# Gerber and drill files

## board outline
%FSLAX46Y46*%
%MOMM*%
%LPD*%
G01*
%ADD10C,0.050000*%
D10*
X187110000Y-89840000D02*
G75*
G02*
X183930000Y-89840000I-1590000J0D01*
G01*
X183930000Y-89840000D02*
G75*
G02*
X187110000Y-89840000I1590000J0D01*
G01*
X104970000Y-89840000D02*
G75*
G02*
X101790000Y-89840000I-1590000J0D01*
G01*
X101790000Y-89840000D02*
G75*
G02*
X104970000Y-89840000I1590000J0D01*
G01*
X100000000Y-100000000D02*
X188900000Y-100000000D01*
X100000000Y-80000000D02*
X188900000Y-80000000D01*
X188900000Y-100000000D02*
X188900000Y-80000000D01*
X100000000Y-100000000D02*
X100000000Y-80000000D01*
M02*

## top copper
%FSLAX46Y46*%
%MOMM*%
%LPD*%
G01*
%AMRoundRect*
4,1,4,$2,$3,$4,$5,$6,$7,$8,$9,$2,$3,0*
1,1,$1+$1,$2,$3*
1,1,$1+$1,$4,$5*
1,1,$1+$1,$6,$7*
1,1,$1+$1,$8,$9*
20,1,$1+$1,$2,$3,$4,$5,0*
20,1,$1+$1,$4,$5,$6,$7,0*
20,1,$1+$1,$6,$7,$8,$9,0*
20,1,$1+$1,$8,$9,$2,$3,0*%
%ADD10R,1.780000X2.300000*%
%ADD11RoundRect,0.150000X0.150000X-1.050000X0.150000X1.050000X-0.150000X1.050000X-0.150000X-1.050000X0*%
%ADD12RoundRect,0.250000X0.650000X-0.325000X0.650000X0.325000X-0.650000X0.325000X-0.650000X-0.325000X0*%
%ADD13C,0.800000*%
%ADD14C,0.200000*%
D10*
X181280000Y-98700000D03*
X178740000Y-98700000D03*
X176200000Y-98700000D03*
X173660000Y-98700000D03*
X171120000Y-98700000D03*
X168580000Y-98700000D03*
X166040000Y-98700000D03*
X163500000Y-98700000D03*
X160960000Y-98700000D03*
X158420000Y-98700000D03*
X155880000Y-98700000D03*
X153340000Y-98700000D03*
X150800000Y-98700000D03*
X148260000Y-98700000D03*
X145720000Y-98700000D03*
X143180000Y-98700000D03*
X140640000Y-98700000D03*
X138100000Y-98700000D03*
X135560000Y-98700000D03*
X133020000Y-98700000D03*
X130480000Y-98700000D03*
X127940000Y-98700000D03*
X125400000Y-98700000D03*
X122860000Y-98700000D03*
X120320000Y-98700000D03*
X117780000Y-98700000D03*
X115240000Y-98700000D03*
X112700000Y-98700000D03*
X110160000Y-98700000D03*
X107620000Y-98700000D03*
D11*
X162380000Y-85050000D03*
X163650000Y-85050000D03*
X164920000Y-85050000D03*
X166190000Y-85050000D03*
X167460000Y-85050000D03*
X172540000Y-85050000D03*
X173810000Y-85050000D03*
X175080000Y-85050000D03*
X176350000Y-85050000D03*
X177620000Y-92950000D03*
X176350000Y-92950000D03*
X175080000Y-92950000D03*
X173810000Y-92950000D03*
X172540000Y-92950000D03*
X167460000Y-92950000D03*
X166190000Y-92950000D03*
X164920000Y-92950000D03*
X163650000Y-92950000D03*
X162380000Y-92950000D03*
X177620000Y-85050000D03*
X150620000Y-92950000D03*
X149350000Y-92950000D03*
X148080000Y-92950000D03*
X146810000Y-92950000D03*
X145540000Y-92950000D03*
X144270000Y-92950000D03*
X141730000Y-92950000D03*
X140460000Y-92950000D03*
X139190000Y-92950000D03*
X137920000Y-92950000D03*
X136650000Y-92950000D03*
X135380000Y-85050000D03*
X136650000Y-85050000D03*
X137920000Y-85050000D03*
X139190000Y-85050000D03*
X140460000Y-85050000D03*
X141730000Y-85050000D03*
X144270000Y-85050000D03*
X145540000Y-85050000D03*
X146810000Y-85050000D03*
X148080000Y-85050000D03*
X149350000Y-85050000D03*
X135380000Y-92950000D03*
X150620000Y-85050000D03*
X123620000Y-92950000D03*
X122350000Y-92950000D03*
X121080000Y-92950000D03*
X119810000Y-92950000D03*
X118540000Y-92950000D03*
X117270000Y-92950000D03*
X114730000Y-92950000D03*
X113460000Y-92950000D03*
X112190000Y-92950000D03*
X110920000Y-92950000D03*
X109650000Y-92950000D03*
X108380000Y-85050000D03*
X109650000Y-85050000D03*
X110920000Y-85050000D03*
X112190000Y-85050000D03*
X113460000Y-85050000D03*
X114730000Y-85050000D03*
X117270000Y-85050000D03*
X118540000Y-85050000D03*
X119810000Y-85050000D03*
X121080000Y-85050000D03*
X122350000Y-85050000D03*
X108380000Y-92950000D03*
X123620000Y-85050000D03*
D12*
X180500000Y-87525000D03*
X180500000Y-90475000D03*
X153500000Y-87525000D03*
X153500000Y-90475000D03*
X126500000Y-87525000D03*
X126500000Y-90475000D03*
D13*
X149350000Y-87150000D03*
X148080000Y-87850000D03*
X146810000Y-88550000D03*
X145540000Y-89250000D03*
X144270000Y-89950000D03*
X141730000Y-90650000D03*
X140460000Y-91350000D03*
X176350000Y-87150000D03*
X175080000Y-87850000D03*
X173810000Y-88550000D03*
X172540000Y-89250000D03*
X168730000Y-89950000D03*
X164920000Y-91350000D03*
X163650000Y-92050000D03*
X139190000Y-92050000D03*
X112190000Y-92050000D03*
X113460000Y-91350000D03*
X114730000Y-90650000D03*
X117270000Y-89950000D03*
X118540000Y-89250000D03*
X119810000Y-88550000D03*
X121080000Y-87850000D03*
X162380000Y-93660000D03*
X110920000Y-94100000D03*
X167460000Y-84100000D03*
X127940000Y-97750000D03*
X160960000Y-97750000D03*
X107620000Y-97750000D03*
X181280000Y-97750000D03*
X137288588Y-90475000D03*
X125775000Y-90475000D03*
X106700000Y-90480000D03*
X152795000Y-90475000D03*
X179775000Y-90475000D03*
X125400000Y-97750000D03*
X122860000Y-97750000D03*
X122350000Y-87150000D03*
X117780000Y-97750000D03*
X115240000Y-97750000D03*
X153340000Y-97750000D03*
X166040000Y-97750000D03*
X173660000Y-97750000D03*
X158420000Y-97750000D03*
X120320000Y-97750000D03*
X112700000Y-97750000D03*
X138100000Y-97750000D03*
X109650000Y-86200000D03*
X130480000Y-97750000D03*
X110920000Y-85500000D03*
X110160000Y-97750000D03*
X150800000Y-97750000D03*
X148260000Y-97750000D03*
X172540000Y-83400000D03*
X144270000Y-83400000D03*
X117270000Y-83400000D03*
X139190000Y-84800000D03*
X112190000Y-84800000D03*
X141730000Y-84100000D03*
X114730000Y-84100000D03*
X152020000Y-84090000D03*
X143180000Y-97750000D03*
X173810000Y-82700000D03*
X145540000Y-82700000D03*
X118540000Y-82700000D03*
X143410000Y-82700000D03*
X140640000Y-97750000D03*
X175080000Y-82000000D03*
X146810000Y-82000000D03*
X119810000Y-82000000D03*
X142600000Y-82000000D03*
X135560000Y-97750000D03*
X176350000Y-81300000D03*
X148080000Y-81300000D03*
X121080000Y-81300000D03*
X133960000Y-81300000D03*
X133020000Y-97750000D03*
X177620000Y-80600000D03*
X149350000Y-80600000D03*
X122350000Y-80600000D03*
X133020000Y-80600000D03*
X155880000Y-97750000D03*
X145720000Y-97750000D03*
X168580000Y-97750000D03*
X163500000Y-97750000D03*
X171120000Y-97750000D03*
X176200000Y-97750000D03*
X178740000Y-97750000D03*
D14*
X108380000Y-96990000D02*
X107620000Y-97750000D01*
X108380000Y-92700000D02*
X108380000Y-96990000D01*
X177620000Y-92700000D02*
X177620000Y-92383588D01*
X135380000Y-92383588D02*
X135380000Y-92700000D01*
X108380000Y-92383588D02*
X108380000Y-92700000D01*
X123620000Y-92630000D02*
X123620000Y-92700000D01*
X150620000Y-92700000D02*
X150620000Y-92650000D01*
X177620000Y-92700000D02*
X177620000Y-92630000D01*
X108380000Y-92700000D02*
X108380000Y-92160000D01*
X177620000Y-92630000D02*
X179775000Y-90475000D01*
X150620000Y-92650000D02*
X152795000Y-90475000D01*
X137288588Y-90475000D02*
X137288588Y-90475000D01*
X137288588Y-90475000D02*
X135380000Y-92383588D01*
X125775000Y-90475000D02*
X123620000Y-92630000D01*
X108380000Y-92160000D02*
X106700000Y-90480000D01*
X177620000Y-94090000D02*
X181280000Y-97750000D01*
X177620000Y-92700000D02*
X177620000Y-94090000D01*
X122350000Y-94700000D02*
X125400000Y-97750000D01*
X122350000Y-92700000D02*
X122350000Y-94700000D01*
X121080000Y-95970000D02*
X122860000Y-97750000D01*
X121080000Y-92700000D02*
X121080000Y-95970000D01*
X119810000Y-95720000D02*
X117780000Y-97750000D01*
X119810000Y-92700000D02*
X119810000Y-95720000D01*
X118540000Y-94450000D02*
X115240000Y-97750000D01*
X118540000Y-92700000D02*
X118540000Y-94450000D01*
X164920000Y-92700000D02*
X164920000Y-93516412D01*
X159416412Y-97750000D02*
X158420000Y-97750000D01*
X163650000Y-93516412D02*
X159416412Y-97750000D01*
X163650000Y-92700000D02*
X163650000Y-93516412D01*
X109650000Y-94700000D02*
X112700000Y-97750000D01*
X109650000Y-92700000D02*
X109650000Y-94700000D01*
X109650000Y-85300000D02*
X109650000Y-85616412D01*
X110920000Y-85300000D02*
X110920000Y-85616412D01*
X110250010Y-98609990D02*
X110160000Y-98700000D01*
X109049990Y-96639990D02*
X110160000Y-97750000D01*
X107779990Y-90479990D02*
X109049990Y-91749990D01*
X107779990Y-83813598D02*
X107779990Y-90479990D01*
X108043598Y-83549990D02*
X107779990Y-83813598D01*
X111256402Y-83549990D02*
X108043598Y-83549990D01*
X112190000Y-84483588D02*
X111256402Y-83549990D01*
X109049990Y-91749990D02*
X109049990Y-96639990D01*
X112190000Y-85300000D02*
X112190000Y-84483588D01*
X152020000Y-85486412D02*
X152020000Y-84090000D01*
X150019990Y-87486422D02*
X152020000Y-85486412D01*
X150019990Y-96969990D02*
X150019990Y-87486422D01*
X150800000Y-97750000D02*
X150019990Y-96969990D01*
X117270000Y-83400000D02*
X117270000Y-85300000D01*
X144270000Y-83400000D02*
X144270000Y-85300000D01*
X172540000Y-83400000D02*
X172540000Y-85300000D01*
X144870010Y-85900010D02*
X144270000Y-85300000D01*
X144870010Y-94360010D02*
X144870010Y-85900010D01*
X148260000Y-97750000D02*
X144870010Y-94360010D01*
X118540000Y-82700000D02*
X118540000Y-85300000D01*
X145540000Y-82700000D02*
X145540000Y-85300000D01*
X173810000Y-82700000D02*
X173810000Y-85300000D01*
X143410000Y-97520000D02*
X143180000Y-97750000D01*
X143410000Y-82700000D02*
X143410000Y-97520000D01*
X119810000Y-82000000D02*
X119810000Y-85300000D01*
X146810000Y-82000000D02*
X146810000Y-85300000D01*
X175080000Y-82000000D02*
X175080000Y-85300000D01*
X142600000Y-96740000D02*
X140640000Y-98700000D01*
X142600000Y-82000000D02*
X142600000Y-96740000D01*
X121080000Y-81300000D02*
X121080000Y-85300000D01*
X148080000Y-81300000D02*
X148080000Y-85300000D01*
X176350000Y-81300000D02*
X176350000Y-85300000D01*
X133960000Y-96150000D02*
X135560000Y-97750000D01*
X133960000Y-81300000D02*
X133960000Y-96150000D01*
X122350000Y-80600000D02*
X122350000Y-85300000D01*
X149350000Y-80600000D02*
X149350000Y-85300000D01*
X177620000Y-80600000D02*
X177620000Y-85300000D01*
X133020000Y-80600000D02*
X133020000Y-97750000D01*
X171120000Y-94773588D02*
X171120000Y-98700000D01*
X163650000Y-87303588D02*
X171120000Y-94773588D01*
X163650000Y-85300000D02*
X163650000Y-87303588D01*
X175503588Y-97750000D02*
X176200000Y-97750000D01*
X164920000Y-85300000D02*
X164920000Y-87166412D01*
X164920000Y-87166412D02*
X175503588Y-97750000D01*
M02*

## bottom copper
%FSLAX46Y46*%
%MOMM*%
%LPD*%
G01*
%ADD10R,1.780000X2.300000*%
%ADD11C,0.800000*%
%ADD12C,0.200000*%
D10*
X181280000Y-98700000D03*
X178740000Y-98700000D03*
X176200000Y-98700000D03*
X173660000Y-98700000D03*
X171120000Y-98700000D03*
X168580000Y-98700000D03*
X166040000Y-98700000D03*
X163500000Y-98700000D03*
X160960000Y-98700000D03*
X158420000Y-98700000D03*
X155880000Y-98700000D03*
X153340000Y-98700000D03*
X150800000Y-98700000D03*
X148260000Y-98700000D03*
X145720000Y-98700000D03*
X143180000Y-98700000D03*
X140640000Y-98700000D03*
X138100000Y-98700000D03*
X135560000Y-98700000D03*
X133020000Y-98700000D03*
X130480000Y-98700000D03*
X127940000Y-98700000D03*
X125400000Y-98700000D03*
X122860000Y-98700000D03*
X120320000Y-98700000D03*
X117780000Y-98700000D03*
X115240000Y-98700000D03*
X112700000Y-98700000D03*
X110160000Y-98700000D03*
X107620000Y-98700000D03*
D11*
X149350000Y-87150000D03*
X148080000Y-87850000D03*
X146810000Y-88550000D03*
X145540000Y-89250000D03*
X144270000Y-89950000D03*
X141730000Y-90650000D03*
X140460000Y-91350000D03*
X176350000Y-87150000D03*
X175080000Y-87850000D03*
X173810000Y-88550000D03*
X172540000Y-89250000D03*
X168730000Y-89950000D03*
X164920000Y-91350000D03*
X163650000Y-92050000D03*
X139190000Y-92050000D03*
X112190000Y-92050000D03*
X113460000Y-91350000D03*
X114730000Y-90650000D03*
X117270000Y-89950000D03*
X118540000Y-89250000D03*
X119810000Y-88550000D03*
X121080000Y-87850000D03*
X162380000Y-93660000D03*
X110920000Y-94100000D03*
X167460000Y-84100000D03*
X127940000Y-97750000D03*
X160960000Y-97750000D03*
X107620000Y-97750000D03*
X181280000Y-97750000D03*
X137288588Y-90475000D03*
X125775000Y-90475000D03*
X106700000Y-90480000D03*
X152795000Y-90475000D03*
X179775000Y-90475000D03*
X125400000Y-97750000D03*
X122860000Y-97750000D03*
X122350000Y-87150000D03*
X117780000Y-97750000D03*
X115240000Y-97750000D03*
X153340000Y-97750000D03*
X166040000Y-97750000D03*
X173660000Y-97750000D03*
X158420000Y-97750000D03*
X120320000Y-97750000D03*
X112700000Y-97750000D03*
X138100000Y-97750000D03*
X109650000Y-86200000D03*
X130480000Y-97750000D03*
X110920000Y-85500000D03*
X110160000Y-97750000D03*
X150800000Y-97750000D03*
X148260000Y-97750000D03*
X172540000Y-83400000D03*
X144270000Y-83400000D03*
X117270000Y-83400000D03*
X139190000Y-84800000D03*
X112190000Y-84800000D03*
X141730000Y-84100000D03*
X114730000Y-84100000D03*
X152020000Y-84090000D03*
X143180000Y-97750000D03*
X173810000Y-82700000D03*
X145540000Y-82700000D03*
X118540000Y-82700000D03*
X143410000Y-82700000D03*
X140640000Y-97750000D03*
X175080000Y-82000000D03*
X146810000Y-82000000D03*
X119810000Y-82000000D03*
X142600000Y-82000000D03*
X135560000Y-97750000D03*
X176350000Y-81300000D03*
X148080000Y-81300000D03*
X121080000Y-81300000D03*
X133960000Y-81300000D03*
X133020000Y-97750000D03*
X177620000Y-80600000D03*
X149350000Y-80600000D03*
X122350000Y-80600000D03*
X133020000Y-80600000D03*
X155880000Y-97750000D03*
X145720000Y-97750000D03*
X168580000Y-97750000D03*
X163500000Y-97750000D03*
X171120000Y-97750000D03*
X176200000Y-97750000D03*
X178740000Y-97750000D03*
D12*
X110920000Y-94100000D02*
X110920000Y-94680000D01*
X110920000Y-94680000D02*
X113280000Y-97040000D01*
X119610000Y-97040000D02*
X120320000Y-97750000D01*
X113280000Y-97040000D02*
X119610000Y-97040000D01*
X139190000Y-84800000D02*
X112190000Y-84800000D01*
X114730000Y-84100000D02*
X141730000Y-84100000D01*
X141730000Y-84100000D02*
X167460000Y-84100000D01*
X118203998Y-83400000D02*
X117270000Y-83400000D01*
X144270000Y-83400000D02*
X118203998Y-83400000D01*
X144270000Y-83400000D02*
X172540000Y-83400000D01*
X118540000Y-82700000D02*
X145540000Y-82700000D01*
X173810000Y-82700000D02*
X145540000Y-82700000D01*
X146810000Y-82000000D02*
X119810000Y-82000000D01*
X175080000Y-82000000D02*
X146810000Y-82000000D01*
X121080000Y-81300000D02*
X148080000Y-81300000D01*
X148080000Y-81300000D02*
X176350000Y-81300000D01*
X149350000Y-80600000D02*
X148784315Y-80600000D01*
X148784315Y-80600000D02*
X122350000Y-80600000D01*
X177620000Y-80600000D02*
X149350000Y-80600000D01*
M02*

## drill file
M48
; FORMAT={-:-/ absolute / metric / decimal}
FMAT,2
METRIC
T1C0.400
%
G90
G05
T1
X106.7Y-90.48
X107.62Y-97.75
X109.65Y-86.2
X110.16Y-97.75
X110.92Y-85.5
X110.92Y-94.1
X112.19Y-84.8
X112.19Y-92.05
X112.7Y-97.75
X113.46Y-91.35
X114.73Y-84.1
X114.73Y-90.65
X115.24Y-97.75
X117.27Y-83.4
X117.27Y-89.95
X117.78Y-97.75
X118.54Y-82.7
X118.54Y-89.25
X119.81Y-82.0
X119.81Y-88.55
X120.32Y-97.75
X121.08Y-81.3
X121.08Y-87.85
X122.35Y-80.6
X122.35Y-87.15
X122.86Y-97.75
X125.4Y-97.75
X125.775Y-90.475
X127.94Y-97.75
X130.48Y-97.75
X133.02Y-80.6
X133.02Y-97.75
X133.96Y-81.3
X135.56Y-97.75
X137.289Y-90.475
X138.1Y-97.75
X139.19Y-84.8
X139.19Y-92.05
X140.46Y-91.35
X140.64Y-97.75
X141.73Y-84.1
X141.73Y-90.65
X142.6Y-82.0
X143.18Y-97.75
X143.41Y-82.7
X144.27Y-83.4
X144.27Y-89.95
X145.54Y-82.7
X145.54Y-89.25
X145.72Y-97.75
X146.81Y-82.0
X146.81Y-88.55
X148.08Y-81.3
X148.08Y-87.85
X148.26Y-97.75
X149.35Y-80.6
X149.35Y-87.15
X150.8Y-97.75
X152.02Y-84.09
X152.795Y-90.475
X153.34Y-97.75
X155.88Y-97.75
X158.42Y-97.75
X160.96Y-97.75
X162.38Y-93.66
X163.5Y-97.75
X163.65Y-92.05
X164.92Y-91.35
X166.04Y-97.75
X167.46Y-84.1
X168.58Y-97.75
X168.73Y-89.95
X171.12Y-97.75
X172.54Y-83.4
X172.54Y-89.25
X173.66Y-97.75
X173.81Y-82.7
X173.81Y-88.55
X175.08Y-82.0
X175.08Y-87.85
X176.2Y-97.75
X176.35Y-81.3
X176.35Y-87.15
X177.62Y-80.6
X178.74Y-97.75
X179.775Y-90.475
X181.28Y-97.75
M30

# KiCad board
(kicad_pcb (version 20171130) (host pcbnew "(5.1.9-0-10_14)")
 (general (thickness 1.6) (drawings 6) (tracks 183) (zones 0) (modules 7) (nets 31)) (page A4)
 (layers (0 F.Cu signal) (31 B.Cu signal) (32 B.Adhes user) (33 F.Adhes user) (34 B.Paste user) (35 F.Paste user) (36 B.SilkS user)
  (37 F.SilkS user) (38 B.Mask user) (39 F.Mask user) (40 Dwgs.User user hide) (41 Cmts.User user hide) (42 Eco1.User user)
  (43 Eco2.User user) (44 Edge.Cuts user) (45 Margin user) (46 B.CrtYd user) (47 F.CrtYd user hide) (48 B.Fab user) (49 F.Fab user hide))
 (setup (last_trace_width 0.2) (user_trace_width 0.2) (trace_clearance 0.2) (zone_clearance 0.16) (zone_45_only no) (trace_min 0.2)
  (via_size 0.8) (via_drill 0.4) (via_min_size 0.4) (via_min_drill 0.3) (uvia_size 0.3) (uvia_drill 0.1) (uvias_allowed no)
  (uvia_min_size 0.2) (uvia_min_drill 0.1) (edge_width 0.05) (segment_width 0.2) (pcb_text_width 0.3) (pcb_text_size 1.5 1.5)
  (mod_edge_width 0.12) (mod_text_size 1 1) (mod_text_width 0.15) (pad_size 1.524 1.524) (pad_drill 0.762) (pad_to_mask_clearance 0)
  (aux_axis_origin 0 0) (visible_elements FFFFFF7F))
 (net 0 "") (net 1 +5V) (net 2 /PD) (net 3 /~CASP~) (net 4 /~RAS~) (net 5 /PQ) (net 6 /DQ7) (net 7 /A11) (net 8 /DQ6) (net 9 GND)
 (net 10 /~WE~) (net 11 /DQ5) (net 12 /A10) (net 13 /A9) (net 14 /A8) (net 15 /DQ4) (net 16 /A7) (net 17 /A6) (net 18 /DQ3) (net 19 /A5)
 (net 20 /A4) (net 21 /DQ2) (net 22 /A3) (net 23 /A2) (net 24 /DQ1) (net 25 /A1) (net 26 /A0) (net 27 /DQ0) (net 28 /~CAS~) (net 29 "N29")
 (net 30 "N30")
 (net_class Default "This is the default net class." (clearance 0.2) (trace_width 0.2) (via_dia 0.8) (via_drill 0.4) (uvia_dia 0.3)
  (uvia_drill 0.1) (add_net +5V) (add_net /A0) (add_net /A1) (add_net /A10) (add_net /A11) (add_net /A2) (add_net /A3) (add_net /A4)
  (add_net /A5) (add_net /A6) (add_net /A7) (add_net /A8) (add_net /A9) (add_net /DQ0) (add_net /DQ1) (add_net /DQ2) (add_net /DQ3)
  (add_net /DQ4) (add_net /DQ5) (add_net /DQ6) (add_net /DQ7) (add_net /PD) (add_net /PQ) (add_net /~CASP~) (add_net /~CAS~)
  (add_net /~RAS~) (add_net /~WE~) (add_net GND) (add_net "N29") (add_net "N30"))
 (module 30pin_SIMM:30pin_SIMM (layer F.Cu) (at 100 100)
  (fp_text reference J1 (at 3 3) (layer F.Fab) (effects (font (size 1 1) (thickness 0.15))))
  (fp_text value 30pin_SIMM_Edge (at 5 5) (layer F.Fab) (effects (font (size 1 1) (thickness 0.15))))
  (pad 30 connect rect (at 81.28 -1.3) (size 1.78 2.3) (layers B.Cu B.Mask) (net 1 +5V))
  (pad 29 connect rect (at 78.74 -1.3) (size 1.78 2.3) (layers B.Cu B.Mask) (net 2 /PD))
  (pad 28 connect rect (at 76.2 -1.3) (size 1.78 2.3) (layers B.Cu B.Mask) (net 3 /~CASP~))
  (pad 27 connect rect (at 73.66 -1.3) (size 1.78 2.3) (layers B.Cu B.Mask) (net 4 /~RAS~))
  (pad 26 connect rect (at 71.12 -1.3) (size 1.78 2.3) (layers B.Cu B.Mask) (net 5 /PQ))
  (pad 25 connect rect (at 68.58 -1.3) (size 1.78 2.3) (layers B.Cu B.Mask) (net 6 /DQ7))
  (pad 24 connect rect (at 66.04 -1.3) (size 1.78 2.3) (layers B.Cu B.Mask) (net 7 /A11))
  (pad 23 connect rect (at 63.5 -1.3) (size 1.78 2.3) (layers B.Cu B.Mask) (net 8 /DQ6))
  (pad 22 connect rect (at 60.96 -1.3) (size 1.78 2.3) (layers B.Cu B.Mask) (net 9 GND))
  (pad 21 connect rect (at 58.42 -1.3) (size 1.78 2.3) (layers B.Cu B.Mask) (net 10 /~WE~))
  (pad 20 connect rect (at 55.88 -1.3) (size 1.78 2.3) (layers B.Cu B.Mask) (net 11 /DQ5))
  (pad 19 connect rect (at 53.34 -1.3) (size 1.78 2.3) (layers B.Cu B.Mask) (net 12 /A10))
  (pad 18 connect rect (at 50.8 -1.3) (size 1.78 2.3) (layers B.Cu B.Mask) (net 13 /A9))
  (pad 17 connect rect (at 48.26 -1.3) (size 1.78 2.3) (layers B.Cu B.Mask) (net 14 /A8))
  (pad 16 connect rect (at 45.72 -1.3) (size 1.78 2.3) (layers B.Cu B.Mask) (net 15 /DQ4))
  (pad 15 connect rect (at 43.18 -1.3) (size 1.78 2.3) (layers B.Cu B.Mask) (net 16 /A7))
  (pad 14 connect rect (at 40.64 -1.3) (size 1.78 2.3) (layers B.Cu B.Mask) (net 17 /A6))
  (pad 13 connect rect (at 38.1 -1.3) (size 1.78 2.3) (layers B.Cu B.Mask) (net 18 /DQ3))
  (pad 12 connect rect (at 35.56 -1.3) (size 1.78 2.3) (layers B.Cu B.Mask) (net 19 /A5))
  (pad 11 connect rect (at 33.02 -1.3) (size 1.78 2.3) (layers B.Cu B.Mask) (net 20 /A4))
  (pad 10 connect rect (at 30.48 -1.3) (size 1.78 2.3) (layers B.Cu B.Mask) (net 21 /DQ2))
  (pad 9 connect rect (at 27.94 -1.3) (size 1.78 2.3) (layers B.Cu B.Mask) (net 9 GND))
  (pad 8 connect rect (at 25.4 -1.3) (size 1.78 2.3) (layers B.Cu B.Mask) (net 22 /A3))
  (pad 7 connect rect (at 22.86 -1.3) (size 1.78 2.3) (layers B.Cu B.Mask) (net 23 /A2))
  (pad 6 connect rect (at 20.32 -1.3) (size 1.78 2.3) (layers B.Cu B.Mask) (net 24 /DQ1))
  (pad 5 connect rect (at 17.78 -1.3) (size 1.78 2.3) (layers B.Cu B.Mask) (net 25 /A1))
  (pad 4 connect rect (at 15.24 -1.3) (size 1.78 2.3) (layers B.Cu B.Mask) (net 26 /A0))
  (pad 3 connect rect (at 12.7 -1.3) (size 1.78 2.3) (layers B.Cu B.Mask) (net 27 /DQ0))
  (pad 2 connect rect (at 10.16 -1.3) (size 1.78 2.3) (layers B.Cu B.Mask) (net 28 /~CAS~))
  (pad 30 connect rect (at 81.28 -1.3) (size 1.78 2.3) (layers F.Cu F.Mask) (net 1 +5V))
  (pad 29 connect rect (at 78.74 -1.3) (size 1.78 2.3) (layers F.Cu F.Mask) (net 2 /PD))
  (pad 28 connect rect (at 76.2 -1.3) (size 1.78 2.3) (layers F.Cu F.Mask) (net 3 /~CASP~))
  (pad 27 connect rect (at 73.66 -1.3) (size 1.78 2.3) (layers F.Cu F.Mask) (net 4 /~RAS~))
  (pad 26 connect rect (at 71.12 -1.3) (size 1.78 2.3) (layers F.Cu F.Mask) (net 5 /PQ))
  (pad 25 connect rect (at 68.58 -1.3) (size 1.78 2.3) (layers F.Cu F.Mask) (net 6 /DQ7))
  (pad 24 connect rect (at 66.04 -1.3) (size 1.78 2.3) (layers F.Cu F.Mask) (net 7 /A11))
  (pad 23 connect rect (at 63.5 -1.3) (size 1.78 2.3) (layers F.Cu F.Mask) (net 8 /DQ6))
  (pad 22 connect rect (at 60.96 -1.3) (size 1.78 2.3) (layers F.Cu F.Mask) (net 9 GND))
  (pad 21 connect rect (at 58.42 -1.3) (size 1.78 2.3) (layers F.Cu F.Mask) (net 10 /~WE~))
  (pad 20 connect rect (at 55.88 -1.3) (size 1.78 2.3) (layers F.Cu F.Mask) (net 11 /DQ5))
  (pad 19 connect rect (at 53.34 -1.3) (size 1.78 2.3) (layers F.Cu F.Mask) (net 12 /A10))
  (pad 18 connect rect (at 50.8 -1.3) (size 1.78 2.3) (layers F.Cu F.Mask) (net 13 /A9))
  (pad 17 connect rect (at 48.26 -1.3) (size 1.78 2.3) (layers F.Cu F.Mask) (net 14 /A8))
  (pad 16 connect rect (at 45.72 -1.3) (size 1.78 2.3) (layers F.Cu F.Mask) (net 15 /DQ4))
  (pad 15 connect rect (at 43.18 -1.3) (size 1.78 2.3) (layers F.Cu F.Mask) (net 16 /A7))
  (pad 14 connect rect (at 40.64 -1.3) (size 1.78 2.3) (layers F.Cu F.Mask) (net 17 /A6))
  (pad 13 connect rect (at 38.1 -1.3) (size 1.78 2.3) (layers F.Cu F.Mask) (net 18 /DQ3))
  (pad 12 connect rect (at 35.56 -1.3) (size 1.78 2.3) (layers F.Cu F.Mask) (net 19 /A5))
  (pad 11 connect rect (at 33.02 -1.3) (size 1.78 2.3) (layers F.Cu F.Mask) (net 20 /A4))
  (pad 10 connect rect (at 30.48 -1.3) (size 1.78 2.3) (layers F.Cu F.Mask) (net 21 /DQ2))
  (pad 9 connect rect (at 27.94 -1.3) (size 1.78 2.3) (layers F.Cu F.Mask) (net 9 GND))
  (pad 8 connect rect (at 25.4 -1.3) (size 1.78 2.3) (layers F.Cu F.Mask) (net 22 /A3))
  (pad 7 connect rect (at 22.86 -1.3) (size 1.78 2.3) (layers F.Cu F.Mask) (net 23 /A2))
  (pad 6 connect rect (at 20.32 -1.3) (size 1.78 2.3) (layers F.Cu F.Mask) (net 24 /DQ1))
  (pad 5 connect rect (at 17.78 -1.3) (size 1.78 2.3) (layers F.Cu F.Mask) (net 25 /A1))
  (pad 4 connect rect (at 15.24 -1.3) (size 1.78 2.3) (layers F.Cu F.Mask) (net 26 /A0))
  (pad 3 connect rect (at 12.7 -1.3) (size 1.78 2.3) (layers F.Cu F.Mask) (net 27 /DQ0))
  (pad 2 connect rect (at 10.16 -1.3) (size 1.78 2.3) (layers F.Cu F.Mask) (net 28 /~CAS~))
  (pad 1 connect rect (at 7.62 -1.3) (size 1.78 2.3) (layers F.Cu F.Mask) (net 1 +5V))
  (pad 1 connect rect (at 7.62 -1.3) (size 1.78 2.3) (layers B.Cu B.Mask) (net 1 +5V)))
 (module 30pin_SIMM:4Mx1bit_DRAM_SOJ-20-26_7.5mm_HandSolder (layer F.Cu) (at 170 89 90)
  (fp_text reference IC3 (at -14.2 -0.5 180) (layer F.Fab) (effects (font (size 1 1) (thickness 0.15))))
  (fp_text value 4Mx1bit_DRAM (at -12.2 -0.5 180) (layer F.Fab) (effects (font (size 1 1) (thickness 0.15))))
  (pad 26 smd roundrect (at 3.7 -7.62 90) (size 2.4 0.6) (drill (offset 0.25 0)) (layers F.Cu F.Paste F.Mask) (roundrect_rratio 0.25)
   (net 9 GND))
  (pad 25 smd roundrect (at 3.7 -6.35 90) (size 2.4 0.6) (drill (offset 0.25 0)) (layers F.Cu F.Paste F.Mask) (roundrect_rratio 0.25)
   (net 5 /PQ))
  (pad 24 smd roundrect (at 3.7 -5.08 90) (size 2.4 0.6) (drill (offset 0.25 0)) (layers F.Cu F.Paste F.Mask) (roundrect_rratio 0.25)
   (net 3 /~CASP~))
  (pad 23 smd roundrect (at 3.7 -3.81 90) (size 2.4 0.6) (drill (offset 0.25 0)) (layers F.Cu F.Paste F.Mask) (roundrect_rratio 0.25)
   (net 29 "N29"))
  (pad 22 smd roundrect (at 3.7 -2.54 90) (size 2.4 0.6) (drill (offset 0.25 0)) (layers F.Cu F.Paste F.Mask) (roundrect_rratio 0.25)
   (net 13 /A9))
  (pad 18 smd roundrect (at 3.7 2.54 90) (size 2.4 0.6) (drill (offset 0.25 0)) (layers F.Cu F.Paste F.Mask) (roundrect_rratio 0.25)
   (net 14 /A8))
  (pad 17 smd roundrect (at 3.7 3.81 90) (size 2.4 0.6) (drill (offset 0.25 0)) (layers F.Cu F.Paste F.Mask) (roundrect_rratio 0.25)
   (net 16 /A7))
  (pad 16 smd roundrect (at 3.7 5.08 90) (size 2.4 0.6) (drill (offset 0.25 0)) (layers F.Cu F.Paste F.Mask) (roundrect_rratio 0.25)
   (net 17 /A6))
  (pad 15 smd roundrect (at 3.7 6.35 90) (size 2.4 0.6) (drill (offset 0.25 0)) (layers F.Cu F.Paste F.Mask) (roundrect_rratio 0.25)
   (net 19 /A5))
  (pad 13 smd roundrect (at -3.7 7.62 90) (size 2.4 0.6) (drill (offset -0.25 0)) (layers F.Cu F.Paste F.Mask) (roundrect_rratio 0.25)
   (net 1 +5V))
  (pad 12 smd roundrect (at -3.7 6.35 90) (size 2.4 0.6) (drill (offset -0.25 0)) (layers F.Cu F.Paste F.Mask) (roundrect_rratio 0.25)
   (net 22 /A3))
  (pad 11 smd roundrect (at -3.7 5.08 90) (size 2.4 0.6) (drill (offset -0.25 0)) (layers F.Cu F.Paste F.Mask) (roundrect_rratio 0.25)
   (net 23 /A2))
  (pad 10 smd roundrect (at -3.7 3.81 90) (size 2.4 0.6) (drill (offset -0.25 0)) (layers F.Cu F.Paste F.Mask) (roundrect_rratio 0.25)
   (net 25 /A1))
  (pad 9 smd roundrect (at -3.7 2.54 90) (size 2.4 0.6) (drill (offset -0.25 0)) (layers F.Cu F.Paste F.Mask) (roundrect_rratio 0.25)
   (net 26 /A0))
  (pad 5 smd roundrect (at -3.7 -2.54 90) (size 2.4 0.6) (drill (offset -0.25 0)) (layers F.Cu F.Paste F.Mask) (roundrect_rratio 0.25)
   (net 12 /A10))
  (pad 4 smd roundrect (at -3.7 -3.81 90) (size 2.4 0.6) (drill (offset -0.25 0)) (layers F.Cu F.Paste F.Mask) (roundrect_rratio 0.25)
   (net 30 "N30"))
  (pad 3 smd roundrect (at -3.7 -5.08 90) (size 2.4 0.6) (drill (offset -0.25 0)) (layers F.Cu F.Paste F.Mask) (roundrect_rratio 0.25)
   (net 4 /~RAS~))
  (pad 2 smd roundrect (at -3.7 -6.35 90) (size 2.4 0.6) (drill (offset -0.25 0)) (layers F.Cu F.Paste F.Mask) (roundrect_rratio 0.25)
   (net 10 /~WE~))
  (pad 1 smd roundrect (at -3.7 -7.62 90) (size 2.4 0.6) (drill (offset -0.25 0)) (layers F.Cu F.Paste F.Mask) (roundrect_rratio 0.25)
   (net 2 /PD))
  (pad 14 smd roundrect (at 3.7 7.62 90) (size 2.4 0.6) (drill (offset 0.25 0)) (layers F.Cu F.Paste F.Mask) (roundrect_rratio 0.25)
   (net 20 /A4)))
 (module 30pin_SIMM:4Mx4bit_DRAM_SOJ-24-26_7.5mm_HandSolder (layer F.Cu) (at 143 89 90)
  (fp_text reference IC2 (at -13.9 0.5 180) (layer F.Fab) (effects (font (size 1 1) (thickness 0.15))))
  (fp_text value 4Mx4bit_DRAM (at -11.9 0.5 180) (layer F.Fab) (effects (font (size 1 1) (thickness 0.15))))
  (pad 13 smd roundrect (at -3.7 7.62 90) (size 2.4 0.6) (drill (offset -0.25 0)) (layers F.Cu F.Paste F.Mask) (roundrect_rratio 0.25)
   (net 1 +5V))
  (pad 12 smd roundrect (at -3.7 6.35 90) (size 2.4 0.6) (drill (offset -0.25 0)) (layers F.Cu F.Paste F.Mask) (roundrect_rratio 0.25)
   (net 22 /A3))
  (pad 11 smd roundrect (at -3.7 5.08 90) (size 2.4 0.6) (drill (offset -0.25 0)) (layers F.Cu F.Paste F.Mask) (roundrect_rratio 0.25)
   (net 23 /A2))
  (pad 10 smd roundrect (at -3.7 3.81 90) (size 2.4 0.6) (drill (offset -0.25 0)) (layers F.Cu F.Paste F.Mask) (roundrect_rratio 0.25)
   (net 25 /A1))
  (pad 9 smd roundrect (at -3.7 2.54 90) (size 2.4 0.6) (drill (offset -0.25 0)) (layers F.Cu F.Paste F.Mask) (roundrect_rratio 0.25)
   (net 26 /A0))
  (pad 8 smd roundrect (at -3.7 1.27 90) (size 2.4 0.6) (drill (offset -0.25 0)) (layers F.Cu F.Paste F.Mask) (roundrect_rratio 0.25)
   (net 12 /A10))
  (pad 6 smd roundrect (at -3.7 -1.27 90) (size 2.4 0.6) (drill (offset -0.25 0)) (layers F.Cu F.Paste F.Mask) (roundrect_rratio 0.25)
   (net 7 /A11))
  (pad 5 smd roundrect (at -3.7 -2.54 90) (size 2.4 0.6) (drill (offset -0.25 0)) (layers F.Cu F.Paste F.Mask) (roundrect_rratio 0.25)
   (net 4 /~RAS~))
  (pad 4 smd roundrect (at -3.7 -3.81 90) (size 2.4 0.6) (drill (offset -0.25 0)) (layers F.Cu F.Paste F.Mask) (roundrect_rratio 0.25)
   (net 10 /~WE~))
  (pad 3 smd roundrect (at -3.7 -5.08 90) (size 2.4 0.6) (drill (offset -0.25 0)) (layers F.Cu F.Paste F.Mask) (roundrect_rratio 0.25)
   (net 11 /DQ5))
  (pad 2 smd roundrect (at -3.7 -6.35 90) (size 2.4 0.6) (drill (offset -0.25 0)) (layers F.Cu F.Paste F.Mask) (roundrect_rratio 0.25)
   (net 15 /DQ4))
  (pad 26 smd roundrect (at 3.7 -7.62 90) (size 2.4 0.6) (drill (offset 0.25 0)) (layers F.Cu F.Paste F.Mask) (roundrect_rratio 0.25)
   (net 9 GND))
  (pad 25 smd roundrect (at 3.7 -6.35 90) (size 2.4 0.6) (drill (offset 0.25 0)) (layers F.Cu F.Paste F.Mask) (roundrect_rratio 0.25)
   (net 6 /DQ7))
  (pad 24 smd roundrect (at 3.7 -5.08 90) (size 2.4 0.6) (drill (offset 0.25 0)) (layers F.Cu F.Paste F.Mask) (roundrect_rratio 0.25)
   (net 8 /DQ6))
  (pad 23 smd roundrect (at 3.7 -3.81 90) (size 2.4 0.6) (drill (offset 0.25 0)) (layers F.Cu F.Paste F.Mask) (roundrect_rratio 0.25)
   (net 28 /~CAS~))
  (pad 22 smd roundrect (at 3.7 -2.54 90) (size 2.4 0.6) (drill (offset 0.25 0)) (layers F.Cu F.Paste F.Mask) (roundrect_rratio 0.25)
   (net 9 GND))
  (pad 21 smd roundrect (at 3.7 -1.27 90) (size 2.4 0.6) (drill (offset 0.25 0)) (layers F.Cu F.Paste F.Mask) (roundrect_rratio 0.25)
   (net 13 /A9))
  (pad 19 smd roundrect (at 3.7 1.27 90) (size 2.4 0.6) (drill (offset 0.25 0)) (layers F.Cu F.Paste F.Mask) (roundrect_rratio 0.25)
   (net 14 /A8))
  (pad 18 smd roundrect (at 3.7 2.54 90) (size 2.4 0.6) (drill (offset 0.25 0)) (layers F.Cu F.Paste F.Mask) (roundrect_rratio 0.25)
   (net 16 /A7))
  (pad 17 smd roundrect (at 3.7 3.81 90) (size 2.4 0.6) (drill (offset 0.25 0)) (layers F.Cu F.Paste F.Mask) (roundrect_rratio 0.25)
   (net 17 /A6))
  (pad 16 smd roundrect (at 3.7 5.08 90) (size 2.4 0.6) (drill (offset 0.25 0)) (layers F.Cu F.Paste F.Mask) (roundrect_rratio 0.25)
   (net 19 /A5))
  (pad 15 smd roundrect (at 3.7 6.35 90) (size 2.4 0.6) (drill (offset 0.25 0)) (layers F.Cu F.Paste F.Mask) (roundrect_rratio 0.25)
   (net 20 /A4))
  (pad 1 smd roundrect (at -3.7 -7.62 90) (size 2.4 0.6) (drill (offset -0.25 0)) (layers F.Cu F.Paste F.Mask) (roundrect_rratio 0.25)
   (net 1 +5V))
  (pad 14 smd roundrect (at 3.7 7.62 90) (size 2.4 0.6) (drill (offset 0.25 0)) (layers F.Cu F.Paste F.Mask) (roundrect_rratio 0.25)
   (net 9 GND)))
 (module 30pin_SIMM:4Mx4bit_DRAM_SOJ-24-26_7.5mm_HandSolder (layer F.Cu) (at 116 89 90)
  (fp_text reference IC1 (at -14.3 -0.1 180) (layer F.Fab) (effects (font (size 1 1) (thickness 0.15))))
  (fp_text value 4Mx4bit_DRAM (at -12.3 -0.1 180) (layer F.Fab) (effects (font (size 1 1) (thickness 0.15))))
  (pad 13 smd roundrect (at -3.7 7.62 90) (size 2.4 0.6) (drill (offset -0.25 0)) (layers F.Cu F.Paste F.Mask) (roundrect_rratio 0.25)
   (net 1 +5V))
  (pad 12 smd roundrect (at -3.7 6.35 90) (size 2.4 0.6) (drill (offset -0.25 0)) (layers F.Cu F.Paste F.Mask) (roundrect_rratio 0.25)
   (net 22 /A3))
  (pad 11 smd roundrect (at -3.7 5.08 90) (size 2.4 0.6) (drill (offset -0.25 0)) (layers F.Cu F.Paste F.Mask) (roundrect_rratio 0.25)
   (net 23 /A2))
  (pad 10 smd roundrect (at -3.7 3.81 90) (size 2.4 0.6) (drill (offset -0.25 0)) (layers F.Cu F.Paste F.Mask) (roundrect_rratio 0.25)
   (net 25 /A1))
  (pad 9 smd roundrect (at -3.7 2.54 90) (size 2.4 0.6) (drill (offset -0.25 0)) (layers F.Cu F.Paste F.Mask) (roundrect_rratio 0.25)
   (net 26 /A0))
  (pad 8 smd roundrect (at -3.7 1.27 90) (size 2.4 0.6) (drill (offset -0.25 0)) (layers F.Cu F.Paste F.Mask) (roundrect_rratio 0.25)
   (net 12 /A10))
  (pad 6 smd roundrect (at -3.7 -1.27 90) (size 2.4 0.6) (drill (offset -0.25 0)) (layers F.Cu F.Paste F.Mask) (roundrect_rratio 0.25)
   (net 7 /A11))
  (pad 5 smd roundrect (at -3.7 -2.54 90) (size 2.4 0.6) (drill (offset -0.25 0)) (layers F.Cu F.Paste F.Mask) (roundrect_rratio 0.25)
   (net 4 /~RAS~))
  (pad 4 smd roundrect (at -3.7 -3.81 90) (size 2.4 0.6) (drill (offset -0.25 0)) (layers F.Cu F.Paste F.Mask) (roundrect_rratio 0.25)
   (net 10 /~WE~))
  (pad 3 smd roundrect (at -3.7 -5.08 90) (size 2.4 0.6) (drill (offset -0.25 0)) (layers F.Cu F.Paste F.Mask) (roundrect_rratio 0.25)
   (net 24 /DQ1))
  (pad 2 smd roundrect (at -3.7 -6.35 90) (size 2.4 0.6) (drill (offset -0.25 0)) (layers F.Cu F.Paste F.Mask) (roundrect_rratio 0.25)
   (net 27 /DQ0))
  (pad 26 smd roundrect (at 3.7 -7.62 90) (size 2.4 0.6) (drill (offset 0.25 0)) (layers F.Cu F.Paste F.Mask) (roundrect_rratio 0.25)
   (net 9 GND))
  (pad 25 smd roundrect (at 3.7 -6.35 90) (size 2.4 0.6) (drill (offset 0.25 0)) (layers F.Cu F.Paste F.Mask) (roundrect_rratio 0.25)
   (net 18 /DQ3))
  (pad 24 smd roundrect (at 3.7 -5.08 90) (size 2.4 0.6) (drill (offset 0.25 0)) (layers F.Cu F.Paste F.Mask) (roundrect_rratio 0.25)
   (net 21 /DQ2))
  (pad 23 smd roundrect (at 3.7 -3.81 90) (size 2.4 0.6) (drill (offset 0.25 0)) (layers F.Cu F.Paste F.Mask) (roundrect_rratio 0.25)
   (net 28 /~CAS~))
  (pad 22 smd roundrect (at 3.7 -2.54 90) (size 2.4 0.6) (drill (offset 0.25 0)) (layers F.Cu F.Paste F.Mask) (roundrect_rratio 0.25)
   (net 9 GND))
  (pad 21 smd roundrect (at 3.7 -1.27 90) (size 2.4 0.6) (drill (offset 0.25 0)) (layers F.Cu F.Paste F.Mask) (roundrect_rratio 0.25)
   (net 13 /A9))
  (pad 19 smd roundrect (at 3.7 1.27 90) (size 2.4 0.6) (drill (offset 0.25 0)) (layers F.Cu F.Paste F.Mask) (roundrect_rratio 0.25)
   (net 14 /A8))
  (pad 18 smd roundrect (at 3.7 2.54 90) (size 2.4 0.6) (drill (offset 0.25 0)) (layers F.Cu F.Paste F.Mask) (roundrect_rratio 0.25)
   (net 16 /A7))
  (pad 17 smd roundrect (at 3.7 3.81 90) (size 2.4 0.6) (drill (offset 0.25 0)) (layers F.Cu F.Paste F.Mask) (roundrect_rratio 0.25)
   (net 17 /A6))
  (pad 16 smd roundrect (at 3.7 5.08 90) (size 2.4 0.6) (drill (offset 0.25 0)) (layers F.Cu F.Paste F.Mask) (roundrect_rratio 0.25)
   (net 19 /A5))
  (pad 15 smd roundrect (at 3.7 6.35 90) (size 2.4 0.6) (drill (offset 0.25 0)) (layers F.Cu F.Paste F.Mask) (roundrect_rratio 0.25)
   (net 20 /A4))
  (pad 1 smd roundrect (at -3.7 -7.62 90) (size 2.4 0.6) (drill (offset -0.25 0)) (layers F.Cu F.Paste F.Mask) (roundrect_rratio 0.25)
   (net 1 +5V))
  (pad 14 smd roundrect (at 3.7 7.62 90) (size 2.4 0.6) (drill (offset 0.25 0)) (layers F.Cu F.Paste F.Mask) (roundrect_rratio 0.25)
   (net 9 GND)))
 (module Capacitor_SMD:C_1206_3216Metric (layer F.Cu) (at 180.5 89 90)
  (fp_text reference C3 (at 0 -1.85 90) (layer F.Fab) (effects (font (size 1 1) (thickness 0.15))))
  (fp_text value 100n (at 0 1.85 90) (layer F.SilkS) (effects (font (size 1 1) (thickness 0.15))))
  (pad 2 smd roundrect (at 1.475 0 90) (size 1.15 1.8) (layers F.Cu F.Paste F.Mask) (roundrect_rratio 0.217391) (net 9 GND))
  (pad 1 smd roundrect (at -1.475 0 90) (size 1.15 1.8) (layers F.Cu F.Paste F.Mask) (roundrect_rratio 0.217391) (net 1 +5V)))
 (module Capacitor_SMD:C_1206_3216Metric (layer F.Cu) (at 153.5 89 90)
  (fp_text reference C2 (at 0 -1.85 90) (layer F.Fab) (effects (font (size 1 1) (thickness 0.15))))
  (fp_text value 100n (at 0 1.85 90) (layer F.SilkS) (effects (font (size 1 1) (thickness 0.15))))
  (pad 2 smd roundrect (at 1.475 0 90) (size 1.15 1.8) (layers F.Cu F.Paste F.Mask) (roundrect_rratio 0.217391) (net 9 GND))
  (pad 1 smd roundrect (at -1.475 0 90) (size 1.15 1.8) (layers F.Cu F.Paste F.Mask) (roundrect_rratio 0.217391) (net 1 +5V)))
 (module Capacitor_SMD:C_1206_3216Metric (layer F.Cu) (at 126.5 89 90)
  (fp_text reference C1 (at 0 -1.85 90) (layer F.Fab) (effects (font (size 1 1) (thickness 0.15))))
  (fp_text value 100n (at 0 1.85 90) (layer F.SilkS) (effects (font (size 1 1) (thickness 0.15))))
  (pad 2 smd roundrect (at 1.475 0 90) (size 1.15 1.8) (layers F.Cu F.Paste F.Mask) (roundrect_rratio 0.217391) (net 9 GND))
  (pad 1 smd roundrect (at -1.475 0 90) (size 1.15 1.8) (layers F.Cu F.Paste F.Mask) (roundrect_rratio 0.217391) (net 1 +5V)))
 (gr_circle (center 185.52 89.84) (end 187.11 89.84) (layer Edge.Cuts) (width 0.05))
 (gr_circle (center 103.38 89.84) (end 104.97 89.84) (layer Edge.Cuts) (width 0.05))
 (gr_line (start 100 100) (end 188.9 100) (layer Edge.Cuts) (width 0.05))
 (gr_line (start 100 80) (end 188.9 80) (layer Edge.Cuts) (width 0.05))
 (gr_line (start 188.9 100) (end 188.9 80) (layer Edge.Cuts) (width 0.05))
 (gr_line (start 100 100) (end 100 80) (layer Edge.Cuts) (width 0.05))
 (via (at 149.35 87.15) (size 0.8) (drill 0.4) (layers F.Cu B.Cu) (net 22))
 (via (at 148.08 87.85) (size 0.8) (drill 0.4) (layers F.Cu B.Cu) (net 23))
 (via (at 146.81 88.55) (size 0.8) (drill 0.4) (layers F.Cu B.Cu) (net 25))
 (via (at 145.54 89.25) (size 0.8) (drill 0.4) (layers F.Cu B.Cu) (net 26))
 (via (at 144.27 89.95) (size 0.8) (drill 0.4) (layers F.Cu B.Cu) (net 12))
 (via (at 141.73 90.65) (size 0.8) (drill 0.4) (layers F.Cu B.Cu) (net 7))
 (via (at 140.46 91.35) (size 0.8) (drill 0.4) (layers F.Cu B.Cu) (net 4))
 (via (at 176.35 87.15) (size 0.8) (drill 0.4) (layers F.Cu B.Cu) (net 22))
 (via (at 175.08 87.85) (size 0.8) (drill 0.4) (layers F.Cu B.Cu) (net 23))
 (via (at 173.81 88.55) (size 0.8) (drill 0.4) (layers F.Cu B.Cu) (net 25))
 (via (at 172.54 89.25) (size 0.8) (drill 0.4) (layers F.Cu B.Cu) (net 26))
 (via (at 168.73 89.95) (size 0.8) (drill 0.4) (layers F.Cu B.Cu) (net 12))
 (via (at 164.92 91.35) (size 0.8) (drill 0.4) (layers F.Cu B.Cu) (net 4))
 (via (at 163.65 92.05) (size 0.8) (drill 0.4) (layers F.Cu B.Cu) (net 10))
 (via (at 139.19 92.05) (size 0.8) (drill 0.4) (layers F.Cu B.Cu) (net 10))
 (via (at 112.19 92.05) (size 0.8) (drill 0.4) (layers F.Cu B.Cu) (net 10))
 (via (at 113.46 91.35) (size 0.8) (drill 0.4) (layers F.Cu B.Cu) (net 4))
 (via (at 114.73 90.65) (size 0.8) (drill 0.4) (layers F.Cu B.Cu) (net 7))
 (via (at 117.27 89.95) (size 0.8) (drill 0.4) (layers F.Cu B.Cu) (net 12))
 (via (at 118.54 89.25) (size 0.8) (drill 0.4) (layers F.Cu B.Cu) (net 26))
 (via (at 119.81 88.55) (size 0.8) (drill 0.4) (layers F.Cu B.Cu) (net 25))
 (via (at 121.08 87.85) (size 0.8) (drill 0.4) (layers F.Cu B.Cu) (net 23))
 (via (at 162.38 93.66) (size 0.8) (drill 0.4) (layers F.Cu B.Cu) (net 2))
 (via (at 110.92 94.1) (size 0.8) (drill 0.4) (layers F.Cu B.Cu) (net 24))
 (via (at 167.46 84.1) (size 0.8) (drill 0.4) (layers F.Cu B.Cu) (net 13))
 (via (at 127.94 97.75) (size 0.8) (drill 0.4) (layers F.Cu B.Cu) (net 9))
 (via (at 160.96 97.75) (size 0.8) (drill 0.4) (layers F.Cu B.Cu) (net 9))
 (via (at 107.62 97.75) (size 0.8) (drill 0.4) (layers F.Cu B.Cu) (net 1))
 (via (at 181.28 97.75) (size 0.8) (drill 0.4) (layers F.Cu B.Cu) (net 1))
 (segment (start 108.38 96.99) (end 107.62 97.75) (width 0.2) (layer F.Cu) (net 1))
 (segment (start 108.38 92.7) (end 108.38 96.99) (width 0.2) (layer F.Cu) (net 1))
 (segment (start 177.62 92.7) (end 177.62 92.383588) (width 0.2) (layer F.Cu) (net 1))
 (segment (start 135.38 92.383588) (end 135.38 92.7) (width 0.2) (layer F.Cu) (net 1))
 (segment (start 108.38 92.383588) (end 108.38 92.7) (width 0.2) (layer F.Cu) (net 1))
 (segment (start 123.62 92.63) (end 123.62 92.7) (width 0.2) (layer F.Cu) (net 1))
 (segment (start 150.62 92.7) (end 150.62 92.65) (width 0.2) (layer F.Cu) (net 1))
 (segment (start 177.62 92.7) (end 177.62 92.63) (width 0.2) (layer F.Cu) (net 1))
 (segment (start 108.38 92.7) (end 108.38 92.16) (width 0.2) (layer F.Cu) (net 1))
 (segment (start 177.62 92.63) (end 179.775 90.475) (width 0.2) (layer F.Cu) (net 1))
 (segment (start 150.62 92.65) (end 152.795 90.475) (width 0.2) (layer F.Cu) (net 1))
 (segment (start 137.288588 90.475) (end 137.288588 90.475) (width 0.2) (layer F.Cu) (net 1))
 (segment (start 137.288588 90.475) (end 135.38 92.383588) (width 0.2) (layer F.Cu) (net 1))
 (via (at 137.288588 90.475) (size 0.8) (drill 0.4) (layers F.Cu B.Cu) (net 1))
 (segment (start 125.775 90.475) (end 123.62 92.63) (width 0.2) (layer F.Cu) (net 1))
 (via (at 125.775 90.475) (size 0.8) (drill 0.4) (layers F.Cu B.Cu) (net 1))
 (segment (start 108.38 92.16) (end 106.7 90.48) (width 0.2) (layer F.Cu) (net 1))
 (via (at 106.7 90.48) (size 0.8) (drill 0.4) (layers F.Cu B.Cu) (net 1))
 (via (at 152.795 90.475) (size 0.8) (drill 0.4) (layers F.Cu B.Cu) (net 1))
 (via (at 179.775 90.475) (size 0.8) (drill 0.4) (layers F.Cu B.Cu) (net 1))
 (segment (start 177.62 94.09) (end 181.28 97.75) (width 0.2) (layer F.Cu) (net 1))
 (segment (start 177.62 92.7) (end 177.62 94.09) (width 0.2) (layer F.Cu) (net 1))
 (via (at 125.4 97.75) (size 0.8) (drill 0.4) (layers F.Cu B.Cu) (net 22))
 (segment (start 122.35 94.7) (end 125.4 97.75) (width 0.2) (layer F.Cu) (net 22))
 (segment (start 122.35 92.7) (end 122.35 94.7) (width 0.2) (layer F.Cu) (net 22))
 (via (at 122.86 97.75) (size 0.8) (drill 0.4) (layers F.Cu B.Cu) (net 23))
 (segment (start 121.08 95.97) (end 122.86 97.75) (width 0.2) (layer F.Cu) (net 23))
 (segment (start 121.08 92.7) (end 121.08 95.97) (width 0.2) (layer F.Cu) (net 23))
 (via (at 122.35 87.15) (size 0.8) (drill 0.4) (layers F.Cu B.Cu) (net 22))
 (via (at 117.78 97.75) (size 0.8) (drill 0.4) (layers F.Cu B.Cu) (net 25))
 (segment (start 119.81 95.72) (end 117.78 97.75) (width 0.2) (layer F.Cu) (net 25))
 (segment (start 119.81 92.7) (end 119.81 95.72) (width 0.2) (layer F.Cu) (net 25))
 (via (at 115.24 97.75) (size 0.8) (drill 0.4) (layers F.Cu B.Cu) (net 26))
 (segment (start 118.54 94.45) (end 115.24 97.75) (width 0.2) (layer F.Cu) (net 26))
 (segment (start 118.54 92.7) (end 118.54 94.45) (width 0.2) (layer F.Cu) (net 26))
 (via (at 153.34 97.75) (size 0.8) (drill 0.4) (layers F.Cu B.Cu) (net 12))
 (via (at 166.04 97.75) (size 0.8) (drill 0.4) (layers F.Cu B.Cu) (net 7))
 (via (at 173.66 97.75) (size 0.8) (drill 0.4) (layers F.Cu B.Cu) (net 4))
 (segment (start 164.92 92.7) (end 164.92 93.516412) (width 0.2) (layer F.Cu) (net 4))
 (via (at 158.42 97.75) (size 0.8) (drill 0.4) (layers F.Cu B.Cu) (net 10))
 (segment (start 159.416412 97.75) (end 158.42 97.75) (width 0.2) (layer F.Cu) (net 10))
 (segment (start 163.65 93.516412) (end 159.416412 97.75) (width 0.2) (layer F.Cu) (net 10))
 (segment (start 163.65 92.7) (end 163.65 93.516412) (width 0.2) (layer F.Cu) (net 10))
 (via (at 120.32 97.75) (size 0.8) (drill 0.4) (layers F.Cu B.Cu) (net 24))
 (segment (start 110.92 94.1) (end 110.92 94.68) (width 0.2) (layer B.Cu) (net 24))
 (segment (start 110.92 94.68) (end 113.28 97.04) (width 0.2) (layer B.Cu) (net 24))
 (segment (start 119.61 97.04) (end 120.32 97.75) (width 0.2) (layer B.Cu) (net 24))
 (segment (start 113.28 97.04) (end 119.61 97.04) (width 0.2) (layer B.Cu) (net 24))
 (via (at 112.7 97.75) (size 0.8) (drill 0.4) (layers F.Cu B.Cu) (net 27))
 (segment (start 109.65 94.7) (end 112.7 97.75) (width 0.2) (layer F.Cu) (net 27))
 (segment (start 109.65 92.7) (end 109.65 94.7) (width 0.2) (layer F.Cu) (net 27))
 (via (at 138.1 97.75) (size 0.8) (drill 0.4) (layers F.Cu B.Cu) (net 18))
 (segment (start 109.65 85.3) (end 109.65 85.616412) (width 0.2) (layer F.Cu) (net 18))
 (via (at 109.65 86.2) (size 0.8) (drill 0.4) (layers F.Cu B.Cu) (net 18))
 (via (at 130.48 97.75) (size 0.8) (drill 0.4) (layers F.Cu B.Cu) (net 21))
 (via (at 110.92 85.5) (size 0.8) (drill 0.4) (layers F.Cu B.Cu) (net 21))
 (segment (start 110.92 85.3) (end 110.92 85.616412) (width 0.2) (layer F.Cu) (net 21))
 (via (at 110.16 97.75) (size 0.8) (drill 0.4) (layers F.Cu B.Cu) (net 28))
 (segment (start 110.25001 98.60999) (end 110.16 98.7) (width 0.2) (layer F.Cu) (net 28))
 (via (at 150.8 97.75) (size 0.8) (drill 0.4) (layers F.Cu B.Cu) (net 13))
 (via (at 148.26 97.75) (size 0.8) (drill 0.4) (layers F.Cu B.Cu) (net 14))
 (via (at 172.54 83.4) (size 0.8) (drill 0.4) (layers F.Cu B.Cu) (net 14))
 (via (at 144.27 83.4) (size 0.8) (drill 0.4) (layers F.Cu B.Cu) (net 14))
 (via (at 117.27 83.4) (size 0.8) (drill 0.4) (layers F.Cu B.Cu) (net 14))
 (via (at 139.19 84.8) (size 0.8) (drill 0.4) (layers F.Cu B.Cu) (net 28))
 (via (at 112.19 84.8) (size 0.8) (drill 0.4) (layers F.Cu B.Cu) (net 28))
 (segment (start 139.19 84.8) (end 112.19 84.8) (width 0.2) (layer B.Cu) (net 28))
 (segment (start 109.04999 96.63999) (end 110.16 97.75) (width 0.2) (layer F.Cu) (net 28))
 (segment (start 107.77999 90.47999) (end 109.04999 91.74999) (width 0.2) (layer F.Cu) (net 28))
 (segment (start 107.77999 83.813598) (end 107.77999 90.47999) (width 0.2) (layer F.Cu) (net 28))
 (segment (start 108.043598 83.54999) (end 107.77999 83.813598) (width 0.2) (layer F.Cu) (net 28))
 (segment (start 111.256402 83.54999) (end 108.043598 83.54999) (width 0.2) (layer F.Cu) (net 28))
 (segment (start 112.19 84.483588) (end 111.256402 83.54999) (width 0.2) (layer F.Cu) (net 28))
 (segment (start 109.04999 91.74999) (end 109.04999 96.63999) (width 0.2) (layer F.Cu) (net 28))
 (segment (start 112.19 85.3) (end 112.19 84.483588) (width 0.2) (layer F.Cu) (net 28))
 (via (at 141.73 84.1) (size 0.8) (drill 0.4) (layers F.Cu B.Cu) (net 13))
 (via (at 114.73 84.1) (size 0.8) (drill 0.4) (layers F.Cu B.Cu) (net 13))
 (segment (start 114.73 84.1) (end 141.73 84.1) (width 0.2) (layer B.Cu) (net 13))
 (segment (start 141.73 84.1) (end 167.46 84.1) (width 0.2) (layer B.Cu) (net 13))
 (via (at 152.02 84.09) (size 0.8) (drill 0.4) (layers F.Cu B.Cu) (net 13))
 (segment (start 152.02 85.486412) (end 152.02 84.09) (width 0.2) (layer F.Cu) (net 13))
 (segment (start 150.01999 87.486422) (end 152.02 85.486412) (width 0.2) (layer F.Cu) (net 13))
 (segment (start 150.01999 96.96999) (end 150.01999 87.486422) (width 0.2) (layer F.Cu) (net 13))
 (segment (start 150.8 97.75) (end 150.01999 96.96999) (width 0.2) (layer F.Cu) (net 13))
 (segment (start 117.27 83.4) (end 117.27 85.3) (width 0.2) (layer F.Cu) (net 14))
 (segment (start 118.203998 83.4) (end 117.27 83.4) (width 0.2) (layer B.Cu) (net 14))
 (segment (start 144.27 83.4) (end 118.203998 83.4) (width 0.2) (layer B.Cu) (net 14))
 (segment (start 144.27 83.4) (end 144.27 85.3) (width 0.2) (layer F.Cu) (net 14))
 (segment (start 172.54 83.4) (end 172.54 85.3) (width 0.2) (layer F.Cu) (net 14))
 (segment (start 144.27 83.4) (end 172.54 83.4) (width 0.2) (layer B.Cu) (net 14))
 (segment (start 144.87001 85.90001) (end 144.27 85.3) (width 0.2) (layer F.Cu) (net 14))
 (segment (start 144.87001 94.36001) (end 144.87001 85.90001) (width 0.2) (layer F.Cu) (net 14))
 (segment (start 148.26 97.75) (end 144.87001 94.36001) (width 0.2) (layer F.Cu) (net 14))
 (via (at 143.18 97.75) (size 0.8) (drill 0.4) (layers F.Cu B.Cu) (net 16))
 (via (at 173.81 82.7) (size 0.8) (drill 0.4) (layers F.Cu B.Cu) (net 16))
 (via (at 145.54 82.7) (size 0.8) (drill 0.4) (layers F.Cu B.Cu) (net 16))
 (via (at 118.54 82.7) (size 0.8) (drill 0.4) (layers F.Cu B.Cu) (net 16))
 (segment (start 118.54 82.7) (end 118.54 85.3) (width 0.2) (layer F.Cu) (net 16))
 (segment (start 118.54 82.7) (end 145.54 82.7) (width 0.2) (layer B.Cu) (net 16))
 (segment (start 145.54 82.7) (end 145.54 85.3) (width 0.2) (layer F.Cu) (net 16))
 (segment (start 173.81 82.7) (end 173.81 85.3) (width 0.2) (layer F.Cu) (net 16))
 (segment (start 173.81 82.7) (end 145.54 82.7) (width 0.2) (layer B.Cu) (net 16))
 (via (at 143.41 82.7) (size 0.8) (drill 0.4) (layers F.Cu B.Cu) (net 16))
 (segment (start 143.41 97.52) (end 143.18 97.75) (width 0.2) (layer F.Cu) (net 16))
 (segment (start 143.41 82.7) (end 143.41 97.52) (width 0.2) (layer F.Cu) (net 16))
 (via (at 140.64 97.75) (size 0.8) (drill 0.4) (layers F.Cu B.Cu) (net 17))
 (via (at 175.08 82) (size 0.8) (drill 0.4) (layers F.Cu B.Cu) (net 17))
 (via (at 146.81 82) (size 0.8) (drill 0.4) (layers F.Cu B.Cu) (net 17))
 (via (at 119.81 82) (size 0.8) (drill 0.4) (layers F.Cu B.Cu) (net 17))
 (segment (start 119.81 82) (end 119.81 85.3) (width 0.2) (layer F.Cu) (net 17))
 (segment (start 146.81 82) (end 119.81 82) (width 0.2) (layer B.Cu) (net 17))
 (segment (start 146.81 82) (end 146.81 85.3) (width 0.2) (layer F.Cu) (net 17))
 (segment (start 175.08 82) (end 175.08 85.3) (width 0.2) (layer F.Cu) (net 17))
 (segment (start 175.08 82) (end 146.81 82) (width 0.2) (layer B.Cu) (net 17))
 (via (at 142.6 82) (size 0.8) (drill 0.4) (layers F.Cu B.Cu) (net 17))
 (segment (start 142.6 96.74) (end 140.64 98.7) (width 0.2) (layer F.Cu) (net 17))
 (segment (start 142.6 82) (end 142.6 96.74) (width 0.2) (layer F.Cu) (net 17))
 (via (at 135.56 97.75) (size 0.8) (drill 0.4) (layers F.Cu B.Cu) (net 19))
 (via (at 176.35 81.3) (size 0.8) (drill 0.4) (layers F.Cu B.Cu) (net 19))
 (via (at 148.08 81.3) (size 0.8) (drill 0.4) (layers F.Cu B.Cu) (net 19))
 (via (at 121.08 81.3) (size 0.8) (drill 0.4) (layers F.Cu B.Cu) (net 19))
 (segment (start 121.08 81.3) (end 121.08 85.3) (width 0.2) (layer F.Cu) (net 19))
 (segment (start 121.08 81.3) (end 148.08 81.3) (width 0.2) (layer B.Cu) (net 19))
 (segment (start 148.08 81.3) (end 148.08 85.3) (width 0.2) (layer F.Cu) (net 19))
 (segment (start 176.35 81.3) (end 176.35 85.3) (width 0.2) (layer F.Cu) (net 19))
 (segment (start 148.08 81.3) (end 176.35 81.3) (width 0.2) (layer B.Cu) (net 19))
 (via (at 133.96 81.3) (size 0.8) (drill 0.4) (layers F.Cu B.Cu) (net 19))
 (segment (start 133.96 96.15) (end 135.56 97.75) (width 0.2) (layer F.Cu) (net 19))
 (segment (start 133.96 81.3) (end 133.96 96.15) (width 0.2) (layer F.Cu) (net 19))
 (via (at 133.02 97.75) (size 0.8) (drill 0.4) (layers F.Cu B.Cu) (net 20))
 (via (at 177.62 80.6) (size 0.8) (drill 0.4) (layers F.Cu B.Cu) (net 20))
 (via (at 149.35 80.6) (size 0.8) (drill 0.4) (layers F.Cu B.Cu) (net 20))
 (via (at 122.35 80.6) (size 0.8) (drill 0.4) (layers F.Cu B.Cu) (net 20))
 (segment (start 122.35 80.6) (end 122.35 85.3) (width 0.2) (layer F.Cu) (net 20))
 (segment (start 149.35 80.6) (end 148.784315 80.6) (width 0.2) (layer B.Cu) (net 20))
 (segment (start 148.784315 80.6) (end 122.35 80.6) (width 0.2) (layer B.Cu) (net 20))
 (segment (start 149.35 80.6) (end 149.35 85.3) (width 0.2) (layer F.Cu) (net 20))
 (segment (start 177.62 80.6) (end 177.62 85.3) (width 0.2) (layer F.Cu) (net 20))
 (segment (start 177.62 80.6) (end 149.35 80.6) (width 0.2) (layer B.Cu) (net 20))
 (via (at 133.02 80.6) (size 0.8) (drill 0.4) (layers F.Cu B.Cu) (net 20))
 (segment (start 133.02 80.6) (end 133.02 97.75) (width 0.2) (layer F.Cu) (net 20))
 (via (at 155.88 97.75) (size 0.8) (drill 0.4) (layers F.Cu B.Cu) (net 11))
 (via (at 145.72 97.75) (size 0.8) (drill 0.4) (layers F.Cu B.Cu) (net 15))
 (via (at 168.58 97.75) (size 0.8) (drill 0.4) (layers F.Cu B.Cu) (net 6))
 (via (at 163.5 97.75) (size 0.8) (drill 0.4) (layers F.Cu B.Cu) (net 8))
 (via (at 171.12 97.75) (size 0.8) (drill 0.4) (layers F.Cu B.Cu) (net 5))
 (segment (start 171.12 94.773588) (end 171.12 98.7) (width 0.2) (layer F.Cu) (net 5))
 (segment (start 163.65 87.303588) (end 171.12 94.773588) (width 0.2) (layer F.Cu) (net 5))
 (segment (start 163.65 85.3) (end 163.65 87.303588) (width 0.2) (layer F.Cu) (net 5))
 (via (at 176.2 97.75) (size 0.8) (drill 0.4) (layers F.Cu B.Cu) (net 3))
 (segment (start 175.503588 97.75) (end 176.2 97.75) (width 0.2) (layer F.Cu) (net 3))
 (segment (start 164.92 85.3) (end 164.92 87.166412) (width 0.2) (layer F.Cu) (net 3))
 (segment (start 164.92 87.166412) (end 175.503588 97.75) (width 0.2) (layer F.Cu) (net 3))
 (via (at 178.74 97.75) (size 0.8) (drill 0.4) (layers F.Cu B.Cu) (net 2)))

